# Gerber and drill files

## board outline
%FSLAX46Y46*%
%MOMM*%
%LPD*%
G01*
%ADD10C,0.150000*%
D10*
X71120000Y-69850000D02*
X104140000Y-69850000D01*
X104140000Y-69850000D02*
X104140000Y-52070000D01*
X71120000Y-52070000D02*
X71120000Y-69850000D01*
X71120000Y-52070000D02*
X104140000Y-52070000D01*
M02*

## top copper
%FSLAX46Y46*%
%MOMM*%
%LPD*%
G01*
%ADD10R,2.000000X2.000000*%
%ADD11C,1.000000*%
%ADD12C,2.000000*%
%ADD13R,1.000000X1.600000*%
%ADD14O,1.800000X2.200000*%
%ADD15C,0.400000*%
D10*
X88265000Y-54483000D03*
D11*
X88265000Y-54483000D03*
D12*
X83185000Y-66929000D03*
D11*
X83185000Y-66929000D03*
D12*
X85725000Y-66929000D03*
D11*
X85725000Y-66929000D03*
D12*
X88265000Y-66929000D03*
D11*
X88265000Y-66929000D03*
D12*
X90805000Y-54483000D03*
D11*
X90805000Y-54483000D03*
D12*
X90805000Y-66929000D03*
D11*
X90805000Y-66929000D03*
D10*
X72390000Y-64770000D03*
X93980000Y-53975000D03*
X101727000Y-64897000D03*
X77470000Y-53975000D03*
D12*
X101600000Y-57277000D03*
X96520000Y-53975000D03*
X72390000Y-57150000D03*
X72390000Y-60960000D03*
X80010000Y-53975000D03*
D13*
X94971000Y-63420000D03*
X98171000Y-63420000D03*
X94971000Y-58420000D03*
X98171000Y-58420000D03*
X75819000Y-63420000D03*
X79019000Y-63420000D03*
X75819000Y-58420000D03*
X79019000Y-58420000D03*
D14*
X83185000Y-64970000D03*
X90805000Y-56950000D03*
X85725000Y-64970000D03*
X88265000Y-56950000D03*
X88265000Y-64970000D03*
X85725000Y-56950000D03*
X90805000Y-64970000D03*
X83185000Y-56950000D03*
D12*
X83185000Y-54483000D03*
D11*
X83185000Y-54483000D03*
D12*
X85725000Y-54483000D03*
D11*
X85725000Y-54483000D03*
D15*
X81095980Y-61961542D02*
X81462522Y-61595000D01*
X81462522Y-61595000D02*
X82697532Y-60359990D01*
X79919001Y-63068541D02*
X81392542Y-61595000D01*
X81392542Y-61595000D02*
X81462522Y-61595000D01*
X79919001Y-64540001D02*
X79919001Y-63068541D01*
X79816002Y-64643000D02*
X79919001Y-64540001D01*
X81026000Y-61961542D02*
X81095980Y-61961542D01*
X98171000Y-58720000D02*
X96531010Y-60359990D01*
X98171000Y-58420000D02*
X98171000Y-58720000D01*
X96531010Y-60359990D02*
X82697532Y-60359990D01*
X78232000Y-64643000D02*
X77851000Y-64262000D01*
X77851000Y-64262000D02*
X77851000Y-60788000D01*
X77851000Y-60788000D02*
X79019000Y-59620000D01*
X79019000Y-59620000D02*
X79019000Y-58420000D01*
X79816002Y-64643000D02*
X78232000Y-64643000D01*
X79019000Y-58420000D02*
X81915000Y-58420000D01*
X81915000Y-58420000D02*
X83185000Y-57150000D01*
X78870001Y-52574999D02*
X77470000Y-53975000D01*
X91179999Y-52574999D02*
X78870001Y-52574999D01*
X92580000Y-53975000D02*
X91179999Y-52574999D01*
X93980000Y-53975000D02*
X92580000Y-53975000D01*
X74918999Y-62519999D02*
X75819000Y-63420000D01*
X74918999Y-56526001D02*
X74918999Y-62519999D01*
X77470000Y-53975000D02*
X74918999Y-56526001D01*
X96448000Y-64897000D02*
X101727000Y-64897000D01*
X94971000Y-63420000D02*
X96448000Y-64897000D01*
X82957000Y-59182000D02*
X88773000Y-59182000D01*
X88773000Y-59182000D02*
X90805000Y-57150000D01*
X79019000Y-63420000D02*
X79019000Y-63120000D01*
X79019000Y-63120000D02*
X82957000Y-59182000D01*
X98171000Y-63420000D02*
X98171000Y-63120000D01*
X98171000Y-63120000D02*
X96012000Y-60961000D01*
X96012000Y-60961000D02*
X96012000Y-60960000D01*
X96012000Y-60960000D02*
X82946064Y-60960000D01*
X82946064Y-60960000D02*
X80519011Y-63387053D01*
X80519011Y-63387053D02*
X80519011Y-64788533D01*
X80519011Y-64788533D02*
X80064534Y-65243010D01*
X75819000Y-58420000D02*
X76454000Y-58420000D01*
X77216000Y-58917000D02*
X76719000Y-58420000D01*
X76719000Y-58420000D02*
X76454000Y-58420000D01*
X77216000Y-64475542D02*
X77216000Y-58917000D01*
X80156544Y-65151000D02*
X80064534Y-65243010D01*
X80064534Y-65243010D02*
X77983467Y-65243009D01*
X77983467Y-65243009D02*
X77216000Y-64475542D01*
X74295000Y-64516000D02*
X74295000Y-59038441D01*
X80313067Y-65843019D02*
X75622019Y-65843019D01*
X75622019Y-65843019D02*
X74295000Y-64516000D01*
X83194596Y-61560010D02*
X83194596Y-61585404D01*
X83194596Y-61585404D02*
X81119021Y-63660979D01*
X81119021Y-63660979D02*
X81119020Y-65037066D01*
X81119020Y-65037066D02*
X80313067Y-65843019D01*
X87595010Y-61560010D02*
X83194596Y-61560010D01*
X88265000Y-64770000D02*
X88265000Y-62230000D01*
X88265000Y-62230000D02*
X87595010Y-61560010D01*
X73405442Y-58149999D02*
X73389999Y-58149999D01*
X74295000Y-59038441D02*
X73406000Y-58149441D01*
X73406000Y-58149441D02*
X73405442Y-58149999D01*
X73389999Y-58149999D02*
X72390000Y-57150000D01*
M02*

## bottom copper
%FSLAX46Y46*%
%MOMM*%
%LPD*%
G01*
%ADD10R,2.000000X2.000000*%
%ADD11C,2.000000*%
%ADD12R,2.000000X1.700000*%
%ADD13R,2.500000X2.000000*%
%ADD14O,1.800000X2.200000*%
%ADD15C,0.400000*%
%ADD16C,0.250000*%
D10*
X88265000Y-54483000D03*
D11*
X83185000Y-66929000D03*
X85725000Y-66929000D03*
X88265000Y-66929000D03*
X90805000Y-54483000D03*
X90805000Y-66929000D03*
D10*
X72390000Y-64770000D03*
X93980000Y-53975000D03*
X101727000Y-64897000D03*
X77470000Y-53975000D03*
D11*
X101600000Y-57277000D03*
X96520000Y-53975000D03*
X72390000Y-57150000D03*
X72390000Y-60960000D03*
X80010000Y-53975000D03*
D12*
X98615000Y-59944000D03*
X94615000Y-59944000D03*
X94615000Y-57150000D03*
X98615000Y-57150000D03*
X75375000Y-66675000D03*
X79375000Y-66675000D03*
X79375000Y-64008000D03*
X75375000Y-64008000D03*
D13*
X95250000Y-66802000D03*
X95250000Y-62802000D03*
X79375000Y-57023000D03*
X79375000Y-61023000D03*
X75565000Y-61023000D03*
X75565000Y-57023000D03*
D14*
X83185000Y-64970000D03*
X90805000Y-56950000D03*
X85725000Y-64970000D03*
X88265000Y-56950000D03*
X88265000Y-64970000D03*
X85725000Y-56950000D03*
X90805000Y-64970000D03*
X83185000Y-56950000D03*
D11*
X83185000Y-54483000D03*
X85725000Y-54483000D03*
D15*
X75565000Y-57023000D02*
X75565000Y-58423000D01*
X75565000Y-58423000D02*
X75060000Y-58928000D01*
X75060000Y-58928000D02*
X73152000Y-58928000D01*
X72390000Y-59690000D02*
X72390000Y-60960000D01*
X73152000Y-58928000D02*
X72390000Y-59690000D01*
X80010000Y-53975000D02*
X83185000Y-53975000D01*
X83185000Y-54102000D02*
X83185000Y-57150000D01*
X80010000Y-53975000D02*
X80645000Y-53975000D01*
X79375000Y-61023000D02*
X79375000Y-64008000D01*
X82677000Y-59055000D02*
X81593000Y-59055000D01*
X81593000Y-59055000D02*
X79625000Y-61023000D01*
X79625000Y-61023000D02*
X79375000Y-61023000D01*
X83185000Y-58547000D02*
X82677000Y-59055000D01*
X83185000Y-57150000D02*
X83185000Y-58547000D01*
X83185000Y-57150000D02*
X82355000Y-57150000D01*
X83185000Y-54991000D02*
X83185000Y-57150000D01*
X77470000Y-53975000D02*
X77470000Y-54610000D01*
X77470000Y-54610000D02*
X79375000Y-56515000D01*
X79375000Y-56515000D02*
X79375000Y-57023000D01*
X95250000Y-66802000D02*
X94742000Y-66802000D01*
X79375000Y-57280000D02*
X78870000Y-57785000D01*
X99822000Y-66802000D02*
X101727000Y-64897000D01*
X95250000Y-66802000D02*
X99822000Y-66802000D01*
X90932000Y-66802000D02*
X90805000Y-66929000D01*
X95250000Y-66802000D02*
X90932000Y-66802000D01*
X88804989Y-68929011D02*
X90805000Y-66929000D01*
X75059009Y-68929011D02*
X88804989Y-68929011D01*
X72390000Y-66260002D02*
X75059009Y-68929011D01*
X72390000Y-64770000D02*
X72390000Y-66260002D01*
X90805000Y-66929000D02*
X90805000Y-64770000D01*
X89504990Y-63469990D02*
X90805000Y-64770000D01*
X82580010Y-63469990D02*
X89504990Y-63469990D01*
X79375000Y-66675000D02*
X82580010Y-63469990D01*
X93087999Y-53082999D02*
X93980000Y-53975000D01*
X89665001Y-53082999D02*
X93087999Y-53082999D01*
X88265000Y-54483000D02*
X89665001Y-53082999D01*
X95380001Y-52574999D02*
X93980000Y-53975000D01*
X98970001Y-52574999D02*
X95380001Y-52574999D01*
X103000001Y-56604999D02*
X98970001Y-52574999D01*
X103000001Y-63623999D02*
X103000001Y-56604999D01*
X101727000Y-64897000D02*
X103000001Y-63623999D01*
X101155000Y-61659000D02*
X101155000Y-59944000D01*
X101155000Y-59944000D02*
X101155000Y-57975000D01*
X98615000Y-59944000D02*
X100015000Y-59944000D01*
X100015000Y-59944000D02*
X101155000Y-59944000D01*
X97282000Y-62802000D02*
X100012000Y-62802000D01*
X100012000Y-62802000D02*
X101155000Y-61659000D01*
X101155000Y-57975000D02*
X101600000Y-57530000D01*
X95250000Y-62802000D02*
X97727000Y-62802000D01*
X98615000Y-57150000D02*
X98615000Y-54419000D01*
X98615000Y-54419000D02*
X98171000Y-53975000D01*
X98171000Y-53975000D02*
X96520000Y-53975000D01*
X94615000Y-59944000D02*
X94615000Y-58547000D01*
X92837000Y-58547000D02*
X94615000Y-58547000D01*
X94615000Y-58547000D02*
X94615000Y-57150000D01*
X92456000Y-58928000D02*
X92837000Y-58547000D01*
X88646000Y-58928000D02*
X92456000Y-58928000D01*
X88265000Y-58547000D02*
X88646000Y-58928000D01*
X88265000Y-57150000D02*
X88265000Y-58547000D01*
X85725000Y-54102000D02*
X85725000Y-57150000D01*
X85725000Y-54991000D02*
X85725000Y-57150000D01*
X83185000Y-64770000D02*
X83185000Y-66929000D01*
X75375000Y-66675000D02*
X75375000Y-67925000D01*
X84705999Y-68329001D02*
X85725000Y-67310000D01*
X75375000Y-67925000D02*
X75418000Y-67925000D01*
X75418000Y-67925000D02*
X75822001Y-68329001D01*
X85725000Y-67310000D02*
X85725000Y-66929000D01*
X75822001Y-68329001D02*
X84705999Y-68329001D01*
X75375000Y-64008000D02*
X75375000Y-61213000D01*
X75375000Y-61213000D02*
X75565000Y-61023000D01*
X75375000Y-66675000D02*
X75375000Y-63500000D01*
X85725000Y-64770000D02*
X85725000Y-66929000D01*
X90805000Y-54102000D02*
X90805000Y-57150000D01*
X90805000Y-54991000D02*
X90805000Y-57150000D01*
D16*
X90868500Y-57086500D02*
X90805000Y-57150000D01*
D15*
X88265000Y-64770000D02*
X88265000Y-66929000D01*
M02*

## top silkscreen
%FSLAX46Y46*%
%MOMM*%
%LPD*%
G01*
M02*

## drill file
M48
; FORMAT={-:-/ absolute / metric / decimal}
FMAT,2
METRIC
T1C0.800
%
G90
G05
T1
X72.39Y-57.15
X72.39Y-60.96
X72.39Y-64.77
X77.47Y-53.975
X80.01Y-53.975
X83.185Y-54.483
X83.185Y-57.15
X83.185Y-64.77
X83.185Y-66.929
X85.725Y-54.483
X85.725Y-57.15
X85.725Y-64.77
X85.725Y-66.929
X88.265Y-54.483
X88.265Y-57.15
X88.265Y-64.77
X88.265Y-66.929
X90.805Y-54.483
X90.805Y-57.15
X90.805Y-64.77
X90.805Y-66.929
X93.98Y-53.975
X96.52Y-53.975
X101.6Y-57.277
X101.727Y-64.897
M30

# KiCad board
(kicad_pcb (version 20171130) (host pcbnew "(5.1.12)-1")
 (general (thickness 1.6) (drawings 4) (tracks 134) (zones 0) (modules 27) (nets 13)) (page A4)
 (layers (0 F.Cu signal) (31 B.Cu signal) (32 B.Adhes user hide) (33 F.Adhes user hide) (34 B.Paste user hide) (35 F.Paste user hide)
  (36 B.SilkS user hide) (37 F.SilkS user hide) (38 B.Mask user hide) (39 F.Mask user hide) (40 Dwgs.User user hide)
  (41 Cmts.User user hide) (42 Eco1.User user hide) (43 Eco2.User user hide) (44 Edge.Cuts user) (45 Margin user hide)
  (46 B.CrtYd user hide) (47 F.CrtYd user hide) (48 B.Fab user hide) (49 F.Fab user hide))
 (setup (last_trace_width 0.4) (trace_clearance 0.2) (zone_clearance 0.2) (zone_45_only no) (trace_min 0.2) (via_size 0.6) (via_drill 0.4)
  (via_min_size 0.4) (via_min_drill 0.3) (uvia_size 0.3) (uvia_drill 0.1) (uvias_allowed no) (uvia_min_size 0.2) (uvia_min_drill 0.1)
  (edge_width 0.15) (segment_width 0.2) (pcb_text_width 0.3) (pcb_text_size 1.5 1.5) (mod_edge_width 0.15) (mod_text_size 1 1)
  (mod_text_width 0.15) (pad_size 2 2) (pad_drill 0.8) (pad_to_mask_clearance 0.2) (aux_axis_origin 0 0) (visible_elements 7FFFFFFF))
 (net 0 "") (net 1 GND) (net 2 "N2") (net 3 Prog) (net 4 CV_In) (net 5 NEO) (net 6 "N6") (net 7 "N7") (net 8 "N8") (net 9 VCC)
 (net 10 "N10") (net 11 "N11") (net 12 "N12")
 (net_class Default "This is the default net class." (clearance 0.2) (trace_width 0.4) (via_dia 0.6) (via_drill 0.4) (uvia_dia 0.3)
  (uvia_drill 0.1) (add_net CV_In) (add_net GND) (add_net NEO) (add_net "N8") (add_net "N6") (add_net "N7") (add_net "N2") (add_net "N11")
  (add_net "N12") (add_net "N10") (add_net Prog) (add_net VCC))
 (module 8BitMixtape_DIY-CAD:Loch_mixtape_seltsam (layer F.Cu) (at 88.265 54.483)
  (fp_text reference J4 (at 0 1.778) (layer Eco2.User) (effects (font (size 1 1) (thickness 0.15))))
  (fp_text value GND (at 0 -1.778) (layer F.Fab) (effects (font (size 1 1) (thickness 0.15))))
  (pad 1 thru_hole rect (at 0 0) (size 2 2) (drill 0.8) (layers B.Cu B.Mask) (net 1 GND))
  (pad "" smd circle (at 0 0) (size 1 1) (layers F.Cu F.Paste F.Mask)))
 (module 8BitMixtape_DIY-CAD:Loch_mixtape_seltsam (layer F.Cu) (at 83.185 66.929)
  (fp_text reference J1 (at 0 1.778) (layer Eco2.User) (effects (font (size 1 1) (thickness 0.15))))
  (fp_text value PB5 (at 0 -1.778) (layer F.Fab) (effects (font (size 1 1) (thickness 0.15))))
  (pad 1 thru_hole circle (at 0 0) (size 2 2) (drill 0.8) (layers B.Cu B.Mask) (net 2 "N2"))
  (pad "" smd circle (at 0 0) (size 1 1) (layers F.Cu F.Paste F.Mask)))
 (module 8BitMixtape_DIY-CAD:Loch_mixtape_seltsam (layer F.Cu) (at 85.725 66.929)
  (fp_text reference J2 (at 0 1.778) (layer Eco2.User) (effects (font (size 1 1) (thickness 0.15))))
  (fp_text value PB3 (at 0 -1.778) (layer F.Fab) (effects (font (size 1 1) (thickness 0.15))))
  (pad 1 thru_hole circle (at 0 0) (size 2 2) (drill 0.8) (layers B.Cu B.Mask) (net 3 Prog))
  (pad "" smd circle (at 0 0) (size 1 1) (layers F.Cu F.Paste F.Mask)))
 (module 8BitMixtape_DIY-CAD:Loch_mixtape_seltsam (layer F.Cu) (at 88.265 66.929)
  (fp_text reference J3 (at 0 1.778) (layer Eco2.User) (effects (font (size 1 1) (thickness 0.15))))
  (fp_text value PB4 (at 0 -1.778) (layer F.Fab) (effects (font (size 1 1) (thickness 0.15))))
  (pad 1 thru_hole circle (at 0 0) (size 2 2) (drill 0.8) (layers B.Cu B.Mask) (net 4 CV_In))
  (pad "" smd circle (at 0 0) (size 1 1) (layers F.Cu F.Paste F.Mask)))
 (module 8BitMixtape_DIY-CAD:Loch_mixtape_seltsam (layer F.Cu) (at 90.805 54.483)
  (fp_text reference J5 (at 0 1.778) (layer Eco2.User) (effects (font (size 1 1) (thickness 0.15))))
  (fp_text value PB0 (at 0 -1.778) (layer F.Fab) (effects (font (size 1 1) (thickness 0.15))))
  (pad 1 thru_hole circle (at 0 0) (size 2 2) (drill 0.8) (layers B.Cu B.Mask) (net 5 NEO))
  (pad "" smd circle (at 0 0) (size 1 1) (layers F.Cu F.Paste F.Mask)))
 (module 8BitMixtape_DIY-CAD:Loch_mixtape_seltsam (layer F.Cu) (at 90.805 66.929)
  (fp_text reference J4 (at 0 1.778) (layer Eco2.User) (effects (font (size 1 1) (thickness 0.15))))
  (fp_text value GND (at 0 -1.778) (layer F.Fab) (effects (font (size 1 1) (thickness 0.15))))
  (pad 1 thru_hole circle (at 0 0) (size 2 2) (drill 0.8) (layers B.Cu B.Mask) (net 1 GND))
  (pad "" smd circle (at 0 0) (size 1 1) (layers F.Cu F.Paste F.Mask)))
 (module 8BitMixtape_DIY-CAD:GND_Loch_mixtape (layer F.Cu) (at 72.39 64.77)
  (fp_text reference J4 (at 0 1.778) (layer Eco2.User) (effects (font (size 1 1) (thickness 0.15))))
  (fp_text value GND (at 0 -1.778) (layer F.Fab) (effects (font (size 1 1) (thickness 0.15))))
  (pad 1 thru_hole rect (at 0 0) (size 2 2) (drill 0.8) (layers *.Cu *.Mask) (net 1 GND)))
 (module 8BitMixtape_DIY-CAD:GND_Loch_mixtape (layer F.Cu) (at 93.98 53.975)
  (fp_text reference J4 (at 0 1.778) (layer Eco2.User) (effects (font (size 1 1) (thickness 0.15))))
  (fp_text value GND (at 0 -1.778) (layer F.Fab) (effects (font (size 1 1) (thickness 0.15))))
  (pad 1 thru_hole rect (at 0 0) (size 2 2) (drill 0.8) (layers *.Cu *.Mask) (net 1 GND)))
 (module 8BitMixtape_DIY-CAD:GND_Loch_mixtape (layer F.Cu) (at 101.727 64.897)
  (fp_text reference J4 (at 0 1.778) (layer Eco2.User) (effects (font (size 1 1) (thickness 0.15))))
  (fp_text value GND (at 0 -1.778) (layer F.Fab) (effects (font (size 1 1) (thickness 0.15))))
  (pad 1 thru_hole rect (at 0 0) (size 2 2) (drill 0.8) (layers *.Cu *.Mask) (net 1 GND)))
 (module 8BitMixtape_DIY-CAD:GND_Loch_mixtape (layer F.Cu) (at 77.47 53.975)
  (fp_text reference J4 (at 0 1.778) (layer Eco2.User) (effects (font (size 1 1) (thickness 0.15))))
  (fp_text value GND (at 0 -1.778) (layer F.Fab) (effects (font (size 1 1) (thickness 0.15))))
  (pad 1 thru_hole rect (at 0 0) (size 2 2) (drill 0.8) (layers *.Cu *.Mask) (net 1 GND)))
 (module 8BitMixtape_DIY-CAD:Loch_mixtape (layer F.Cu) (at 101.6 57.277)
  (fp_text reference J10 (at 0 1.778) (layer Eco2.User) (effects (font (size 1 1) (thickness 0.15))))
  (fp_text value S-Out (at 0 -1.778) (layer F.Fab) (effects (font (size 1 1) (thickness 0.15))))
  (pad 1 thru_hole circle (at 0 0) (size 2 2) (drill 0.8) (layers *.Cu *.Mask) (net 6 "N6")))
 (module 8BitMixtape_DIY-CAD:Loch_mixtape (layer F.Cu) (at 96.52 53.975)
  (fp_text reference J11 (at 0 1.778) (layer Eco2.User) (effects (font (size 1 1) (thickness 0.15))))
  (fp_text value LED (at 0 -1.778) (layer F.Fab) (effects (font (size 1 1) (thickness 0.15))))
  (pad 1 thru_hole circle (at 0 0) (size 2 2) (drill 0.8) (layers *.Cu *.Mask) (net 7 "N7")))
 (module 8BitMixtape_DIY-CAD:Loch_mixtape (layer F.Cu) (at 72.39 57.15)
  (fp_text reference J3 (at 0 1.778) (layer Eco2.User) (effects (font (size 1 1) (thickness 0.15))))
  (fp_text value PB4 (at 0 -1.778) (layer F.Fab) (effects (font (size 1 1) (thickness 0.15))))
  (pad 1 thru_hole circle (at 0 0) (size 2 2) (drill 0.8) (layers *.Cu *.Mask) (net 4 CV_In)))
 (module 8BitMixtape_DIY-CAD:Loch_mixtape (layer F.Cu) (at 72.39 60.96)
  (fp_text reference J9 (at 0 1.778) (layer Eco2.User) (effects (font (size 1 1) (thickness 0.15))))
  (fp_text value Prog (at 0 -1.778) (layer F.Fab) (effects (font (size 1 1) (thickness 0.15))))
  (pad 1 thru_hole circle (at 0 0) (size 2 2) (drill 0.8) (layers *.Cu *.Mask) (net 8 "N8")))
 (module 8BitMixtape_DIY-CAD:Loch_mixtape (layer F.Cu) (at 80.01 53.975)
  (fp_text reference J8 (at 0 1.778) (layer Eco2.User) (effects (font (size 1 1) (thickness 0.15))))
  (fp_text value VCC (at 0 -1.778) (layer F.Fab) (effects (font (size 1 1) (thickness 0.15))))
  (pad 1 thru_hole circle (at 0 0) (size 2 2) (drill 0.8) (layers *.Cu *.Mask) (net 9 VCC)))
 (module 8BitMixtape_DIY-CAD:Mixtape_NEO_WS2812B (layer F.Cu) (at 96.571 60.92 270)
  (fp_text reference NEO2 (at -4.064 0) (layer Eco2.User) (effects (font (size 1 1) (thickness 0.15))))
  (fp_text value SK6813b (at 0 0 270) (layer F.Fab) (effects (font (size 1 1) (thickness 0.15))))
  (pad 3 smd rect (at 2.5 1.6 270) (size 1.6 1) (layers F.Cu F.Paste F.Mask) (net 1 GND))
  (pad 4 smd rect (at 2.5 -1.6 270) (size 1.6 1) (layers F.Cu F.Paste F.Mask) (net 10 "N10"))
  (pad 2 smd rect (at -2.5 1.6 270) (size 1.6 1) (layers F.Cu F.Paste F.Mask))
  (pad 1 smd rect (at -2.5 -1.6 270) (size 1.6 1) (layers F.Cu F.Paste F.Mask) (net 9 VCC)))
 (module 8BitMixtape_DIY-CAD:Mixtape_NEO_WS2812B (layer F.Cu) (at 77.419 60.92 270)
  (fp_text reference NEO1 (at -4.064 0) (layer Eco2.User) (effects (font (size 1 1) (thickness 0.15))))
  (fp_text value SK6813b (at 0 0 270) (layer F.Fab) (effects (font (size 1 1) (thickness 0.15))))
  (pad 3 smd rect (at 2.5 1.6 270) (size 1.6 1) (layers F.Cu F.Paste F.Mask) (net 1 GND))
  (pad 4 smd rect (at 2.5 -1.6 270) (size 1.6 1) (layers F.Cu F.Paste F.Mask) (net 5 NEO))
  (pad 2 smd rect (at -2.5 1.6 270) (size 1.6 1) (layers F.Cu F.Paste F.Mask) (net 10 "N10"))
  (pad 1 smd rect (at -2.5 -1.6 270) (size 1.6 1) (layers F.Cu F.Paste F.Mask) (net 9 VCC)))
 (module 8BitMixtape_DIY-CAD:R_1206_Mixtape (layer B.Cu) (at 96.615 59.944 180)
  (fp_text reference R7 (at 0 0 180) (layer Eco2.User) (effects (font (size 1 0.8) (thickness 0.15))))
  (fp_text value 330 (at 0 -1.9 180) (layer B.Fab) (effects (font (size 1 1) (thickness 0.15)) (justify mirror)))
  (pad 1 smd rect (at -2 0 180) (size 2 1.7) (layers B.Cu B.Paste B.Mask) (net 6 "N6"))
  (pad 2 smd rect (at 2 0 180) (size 2 1.7) (layers B.Cu B.Paste B.Mask) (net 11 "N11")))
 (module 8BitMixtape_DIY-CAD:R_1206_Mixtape (layer B.Cu) (at 96.615 57.15)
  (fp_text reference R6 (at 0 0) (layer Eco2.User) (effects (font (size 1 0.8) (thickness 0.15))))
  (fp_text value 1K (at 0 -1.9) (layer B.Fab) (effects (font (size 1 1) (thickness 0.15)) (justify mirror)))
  (pad 1 smd rect (at -2 0) (size 2 1.7) (layers B.Cu B.Paste B.Mask) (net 11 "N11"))
  (pad 2 smd rect (at 2 0) (size 2 1.7) (layers B.Cu B.Paste B.Mask) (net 7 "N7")))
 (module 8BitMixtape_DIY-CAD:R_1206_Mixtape (layer B.Cu) (at 77.375 66.675)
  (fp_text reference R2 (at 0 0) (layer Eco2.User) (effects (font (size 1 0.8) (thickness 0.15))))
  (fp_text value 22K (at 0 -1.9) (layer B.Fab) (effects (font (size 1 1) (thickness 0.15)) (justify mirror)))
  (pad 1 smd rect (at -2 0) (size 2 1.7) (layers B.Cu B.Paste B.Mask) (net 3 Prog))
  (pad 2 smd rect (at 2 0) (size 2 1.7) (layers B.Cu B.Paste B.Mask) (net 1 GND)))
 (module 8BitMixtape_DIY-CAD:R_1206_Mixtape (layer B.Cu) (at 77.375 64.008 180)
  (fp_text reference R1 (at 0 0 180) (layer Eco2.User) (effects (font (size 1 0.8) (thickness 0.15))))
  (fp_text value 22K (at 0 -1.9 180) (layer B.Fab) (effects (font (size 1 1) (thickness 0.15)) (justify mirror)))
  (pad 1 smd rect (at -2 0 180) (size 2 1.7) (layers B.Cu B.Paste B.Mask) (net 9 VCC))
  (pad 2 smd rect (at 2 0 180) (size 2 1.7) (layers B.Cu B.Paste B.Mask) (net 3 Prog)))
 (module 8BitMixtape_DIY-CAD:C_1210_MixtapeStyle (layer B.Cu) (at 95.25 64.802 90)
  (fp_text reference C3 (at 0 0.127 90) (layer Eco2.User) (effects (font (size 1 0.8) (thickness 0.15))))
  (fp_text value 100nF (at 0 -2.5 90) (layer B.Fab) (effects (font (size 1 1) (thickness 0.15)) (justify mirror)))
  (pad 1 smd rect (at -2 0 90) (size 2 2.5) (layers B.Cu B.Paste B.Mask) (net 1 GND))
  (pad 2 smd rect (at 2 0 90) (size 2 2.5) (layers B.Cu B.Paste B.Mask) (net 6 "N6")))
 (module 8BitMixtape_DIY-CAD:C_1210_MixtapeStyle (layer B.Cu) (at 79.375 59.023 270)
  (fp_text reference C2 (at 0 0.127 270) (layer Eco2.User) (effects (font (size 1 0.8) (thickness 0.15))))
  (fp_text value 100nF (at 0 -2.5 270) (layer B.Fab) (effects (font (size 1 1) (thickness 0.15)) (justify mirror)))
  (pad 1 smd rect (at -2 0 270) (size 2 2.5) (layers B.Cu B.Paste B.Mask) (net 1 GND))
  (pad 2 smd rect (at 2 0 270) (size 2 2.5) (layers B.Cu B.Paste B.Mask) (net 9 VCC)))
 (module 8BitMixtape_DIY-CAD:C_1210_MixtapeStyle (layer B.Cu) (at 75.565 59.023 90)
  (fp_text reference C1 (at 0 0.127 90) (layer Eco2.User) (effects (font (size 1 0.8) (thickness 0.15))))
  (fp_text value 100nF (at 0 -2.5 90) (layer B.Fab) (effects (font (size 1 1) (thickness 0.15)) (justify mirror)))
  (pad 1 smd rect (at -2 0 90) (size 2 2.5) (layers B.Cu B.Paste B.Mask) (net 3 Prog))
  (pad 2 smd rect (at 2 0 90) (size 2 2.5) (layers B.Cu B.Paste B.Mask) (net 8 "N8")))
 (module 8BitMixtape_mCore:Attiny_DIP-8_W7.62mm (layer F.Cu) (at 83.185 64.77 90)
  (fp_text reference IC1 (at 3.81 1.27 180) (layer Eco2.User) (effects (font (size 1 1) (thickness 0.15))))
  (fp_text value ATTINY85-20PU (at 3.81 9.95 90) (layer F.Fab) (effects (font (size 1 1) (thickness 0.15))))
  (pad 1 thru_hole oval (at 0 0 90) (size 2.2 1.8) (drill 0.8 (offset -0.2 0)) (layers *.Cu *.Mask) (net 2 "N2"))
  (pad 5 thru_hole oval (at 7.62 7.62 90) (size 2.2 1.8) (drill 0.8 (offset 0.2 0)) (layers *.Cu *.Mask) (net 5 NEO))
  (pad 2 thru_hole oval (at 0 2.54 90) (size 2.2 1.8) (drill 0.8 (offset -0.2 0)) (layers *.Cu *.Mask) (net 3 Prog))
  (pad 6 thru_hole oval (at 7.62 5.08 90) (size 2.2 1.8) (drill 0.8 (offset 0.2 0)) (layers *.Cu *.Mask) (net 11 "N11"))
  (pad 3 thru_hole oval (at 0 5.08 90) (size 2.2 1.8) (drill 0.8 (offset -0.2 0)) (layers *.Cu *.Mask) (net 4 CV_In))
  (pad 7 thru_hole oval (at 7.62 2.54 90) (size 2.2 1.8) (drill 0.8 (offset 0.2 0)) (layers *.Cu *.Mask) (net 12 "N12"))
  (pad 4 thru_hole oval (at 0 7.62 90) (size 2.2 1.8) (drill 0.8 (offset -0.2 0)) (layers *.Cu *.Mask) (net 1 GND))
  (pad 8 thru_hole oval (at 7.62 0 90) (size 2.2 1.8) (drill 0.8 (offset 0.2 0)) (layers *.Cu *.Mask) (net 9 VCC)))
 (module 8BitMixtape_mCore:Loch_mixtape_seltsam (layer F.Cu) (at 83.185 54.483)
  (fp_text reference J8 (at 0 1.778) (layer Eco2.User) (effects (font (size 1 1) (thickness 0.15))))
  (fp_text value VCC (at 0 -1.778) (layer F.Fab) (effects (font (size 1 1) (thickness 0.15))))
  (pad 1 thru_hole circle (at 0 0) (size 2 2) (drill 0.8) (layers B.Cu B.Mask) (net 9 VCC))
  (pad "" smd circle (at 0 0) (size 1 1) (layers F.Cu F.Paste F.Mask)))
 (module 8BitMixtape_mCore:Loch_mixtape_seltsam (layer F.Cu) (at 85.725 54.483)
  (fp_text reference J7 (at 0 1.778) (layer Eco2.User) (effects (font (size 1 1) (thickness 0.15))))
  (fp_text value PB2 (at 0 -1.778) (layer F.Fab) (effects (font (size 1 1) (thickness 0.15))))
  (pad 1 thru_hole circle (at 0 0) (size 2 2) (drill 0.8) (layers B.Cu B.Mask) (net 12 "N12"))
  (pad "" smd circle (at 0 0) (size 1 1) (layers F.Cu F.Paste F.Mask)))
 (gr_line (start 71.12 69.85) (end 104.14 69.85) (layer Edge.Cuts) (width 0.15))
 (gr_line (start 104.14 69.85) (end 104.14 52.07) (layer Edge.Cuts) (width 0.15))
 (gr_line (start 71.12 52.07) (end 71.12 69.85) (layer Edge.Cuts) (width 0.15))
 (gr_line (start 71.12 52.07) (end 104.14 52.07) (layer Edge.Cuts) (width 0.15))
 (segment (start 75.565 57.023) (end 75.565 58.423) (width 0.4) (layer B.Cu) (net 8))
 (segment (start 75.565 58.423) (end 75.06 58.928) (width 0.4) (layer B.Cu) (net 8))
 (segment (start 75.06 58.928) (end 73.152 58.928) (width 0.4) (layer B.Cu) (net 8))
 (segment (start 72.39 59.69) (end 72.39 60.96) (width 0.4) (layer B.Cu) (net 8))
 (segment (start 73.152 58.928) (end 72.39 59.69) (width 0.4) (layer B.Cu) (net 8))
 (segment (start 81.09598 61.961542) (end 81.462522 61.595) (width 0.4) (layer F.Cu) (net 9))
 (segment (start 81.462522 61.595) (end 82.697532 60.35999) (width 0.4) (layer F.Cu) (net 9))
 (segment (start 79.919001 63.068541) (end 81.392542 61.595) (width 0.4) (layer F.Cu) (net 9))
 (segment (start 81.392542 61.595) (end 81.462522 61.595) (width 0.4) (layer F.Cu) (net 9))
 (segment (start 79.919001 64.540001) (end 79.919001 63.068541) (width 0.4) (layer F.Cu) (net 9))
 (segment (start 79.816002 64.643) (end 79.919001 64.540001) (width 0.4) (layer F.Cu) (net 9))
 (segment (start 81.026 61.961542) (end 81.09598 61.961542) (width 0.4) (layer F.Cu) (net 9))
 (segment (start 98.171 58.72) (end 96.53101 60.35999) (width 0.4) (layer F.Cu) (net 9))
 (segment (start 98.171 58.42) (end 98.171 58.72) (width 0.4) (layer F.Cu) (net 9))
 (segment (start 96.53101 60.35999) (end 82.697532 60.35999) (width 0.4) (layer F.Cu) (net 9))
 (segment (start 78.232 64.643) (end 77.851 64.262) (width 0.4) (layer F.Cu) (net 9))
 (segment (start 77.851 64.262) (end 77.851 60.788) (width 0.4) (layer F.Cu) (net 9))
 (segment (start 77.851 60.788) (end 79.019 59.62) (width 0.4) (layer F.Cu) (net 9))
 (segment (start 79.019 59.62) (end 79.019 58.42) (width 0.4) (layer F.Cu) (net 9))
 (segment (start 79.816002 64.643) (end 78.232 64.643) (width 0.4) (layer F.Cu) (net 9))
 (segment (start 79.019 58.42) (end 81.915 58.42) (width 0.4) (layer F.Cu) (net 9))
 (segment (start 81.915 58.42) (end 83.185 57.15) (width 0.4) (layer F.Cu) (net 9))
 (segment (start 80.01 53.975) (end 83.185 53.975) (width 0.4) (layer B.Cu) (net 9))
 (segment (start 83.185 54.102) (end 83.185 57.15) (width 0.4) (layer B.Cu) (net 9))
 (segment (start 80.01 53.975) (end 80.645 53.975) (width 0.4) (layer B.Cu) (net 9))
 (segment (start 79.375 61.023) (end 79.375 64.008) (width 0.4) (layer B.Cu) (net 9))
 (segment (start 82.677 59.055) (end 81.593 59.055) (width 0.4) (layer B.Cu) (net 9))
 (segment (start 81.593 59.055) (end 79.625 61.023) (width 0.4) (layer B.Cu) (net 9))
 (segment (start 79.625 61.023) (end 79.375 61.023) (width 0.4) (layer B.Cu) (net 9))
 (segment (start 83.185 58.547) (end 82.677 59.055) (width 0.4) (layer B.Cu) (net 9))
 (segment (start 83.185 57.15) (end 83.185 58.547) (width 0.4) (layer B.Cu) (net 9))
 (segment (start 83.185 57.15) (end 82.355 57.15) (width 0.4) (layer B.Cu) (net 9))
 (segment (start 83.185 54.991) (end 83.185 57.15) (width 0.4) (layer B.Cu) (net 9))
 (segment (start 77.47 53.975) (end 77.47 54.61) (width 0.4) (layer B.Cu) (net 1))
 (segment (start 77.47 54.61) (end 79.375 56.515) (width 0.4) (layer B.Cu) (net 1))
 (segment (start 79.375 56.515) (end 79.375 57.023) (width 0.4) (layer B.Cu) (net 1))
 (segment (start 95.25 66.802) (end 94.742 66.802) (width 0.4) (layer B.Cu) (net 1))
 (segment (start 79.375 57.28) (end 78.87 57.785) (width 0.4) (layer B.Cu) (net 1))
 (segment (start 78.870001 52.574999) (end 77.47 53.975) (width 0.4) (layer F.Cu) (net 1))
 (segment (start 91.179999 52.574999) (end 78.870001 52.574999) (width 0.4) (layer F.Cu) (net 1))
 (segment (start 92.58 53.975) (end 91.179999 52.574999) (width 0.4) (layer F.Cu) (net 1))
 (segment (start 93.98 53.975) (end 92.58 53.975) (width 0.4) (layer F.Cu) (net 1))
 (segment (start 74.918999 62.519999) (end 75.819 63.42) (width 0.4) (layer F.Cu) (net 1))
 (segment (start 74.918999 56.526001) (end 74.918999 62.519999) (width 0.4) (layer F.Cu) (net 1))
 (segment (start 77.47 53.975) (end 74.918999 56.526001) (width 0.4) (layer F.Cu) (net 1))
 (segment (start 96.448 64.897) (end 101.727 64.897) (width 0.4) (layer F.Cu) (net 1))
 (segment (start 94.971 63.42) (end 96.448 64.897) (width 0.4) (layer F.Cu) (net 1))
 (segment (start 99.822 66.802) (end 101.727 64.897) (width 0.4) (layer B.Cu) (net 1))
 (segment (start 95.25 66.802) (end 99.822 66.802) (width 0.4) (layer B.Cu) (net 1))
 (segment (start 90.932 66.802) (end 90.805 66.929) (width 0.4) (layer B.Cu) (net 1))
 (segment (start 95.25 66.802) (end 90.932 66.802) (width 0.4) (layer B.Cu) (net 1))
 (segment (start 88.804989 68.929011) (end 90.805 66.929) (width 0.4) (layer B.Cu) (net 1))
 (segment (start 75.059009 68.929011) (end 88.804989 68.929011) (width 0.4) (layer B.Cu) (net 1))
 (segment (start 72.39 66.260002) (end 75.059009 68.929011) (width 0.4) (layer B.Cu) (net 1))
 (segment (start 72.39 64.77) (end 72.39 66.260002) (width 0.4) (layer B.Cu) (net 1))
 (segment (start 90.805 66.929) (end 90.805 64.77) (width 0.4) (layer B.Cu) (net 1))
 (segment (start 89.50499 63.46999) (end 90.805 64.77) (width 0.4) (layer B.Cu) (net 1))
 (segment (start 82.58001 63.46999) (end 89.50499 63.46999) (width 0.4) (layer B.Cu) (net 1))
 (segment (start 79.375 66.675) (end 82.58001 63.46999) (width 0.4) (layer B.Cu) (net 1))
 (segment (start 93.087999 53.082999) (end 93.98 53.975) (width 0.4) (layer B.Cu) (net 1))
 (segment (start 89.665001 53.082999) (end 93.087999 53.082999) (width 0.4) (layer B.Cu) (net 1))
 (segment (start 88.265 54.483) (end 89.665001 53.082999) (width 0.4) (layer B.Cu) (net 1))
 (segment (start 95.380001 52.574999) (end 93.98 53.975) (width 0.4) (layer B.Cu) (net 1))
 (segment (start 98.970001 52.574999) (end 95.380001 52.574999) (width 0.4) (layer B.Cu) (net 1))
 (segment (start 103.000001 56.604999) (end 98.970001 52.574999) (width 0.4) (layer B.Cu) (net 1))
 (segment (start 103.000001 63.623999) (end 103.000001 56.604999) (width 0.4) (layer B.Cu) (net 1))
 (segment (start 101.727 64.897) (end 103.000001 63.623999) (width 0.4) (layer B.Cu) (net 1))
 (segment (start 101.155 61.659) (end 101.155 59.944) (width 0.4) (layer B.Cu) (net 6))
 (segment (start 101.155 59.944) (end 101.155 57.975) (width 0.4) (layer B.Cu) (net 6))
 (segment (start 98.615 59.944) (end 100.015 59.944) (width 0.4) (layer B.Cu) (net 6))
 (segment (start 100.015 59.944) (end 101.155 59.944) (width 0.4) (layer B.Cu) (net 6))
 (segment (start 97.282 62.802) (end 100.012 62.802) (width 0.4) (layer B.Cu) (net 6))
 (segment (start 100.012 62.802) (end 101.155 61.659) (width 0.4) (layer B.Cu) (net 6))
 (segment (start 101.155 57.975) (end 101.6 57.53) (width 0.4) (layer B.Cu) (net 6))
 (segment (start 95.25 62.802) (end 97.727 62.802) (width 0.4) (layer B.Cu) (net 6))
 (segment (start 98.615 57.15) (end 98.615 54.419) (width 0.4) (layer B.Cu) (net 7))
 (segment (start 98.615 54.419) (end 98.171 53.975) (width 0.4) (layer B.Cu) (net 7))
 (segment (start 98.171 53.975) (end 96.52 53.975) (width 0.4) (layer B.Cu) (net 7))
 (segment (start 94.615 59.944) (end 94.615 58.547) (width 0.4) (layer B.Cu) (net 11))
 (segment (start 92.837 58.547) (end 94.615 58.547) (width 0.4) (layer B.Cu) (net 11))
 (segment (start 94.615 58.547) (end 94.615 57.15) (width 0.4) (layer B.Cu) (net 11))
 (segment (start 92.456 58.928) (end 92.837 58.547) (width 0.4) (layer B.Cu) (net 11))
 (segment (start 88.646 58.928) (end 92.456 58.928) (width 0.4) (layer B.Cu) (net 11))
 (segment (start 88.265 58.547) (end 88.646 58.928) (width 0.4) (layer B.Cu) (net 11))
 (segment (start 88.265 57.15) (end 88.265 58.547) (width 0.4) (layer B.Cu) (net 11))
 (segment (start 85.725 54.102) (end 85.725 57.15) (width 0.4) (layer B.Cu) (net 12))
 (segment (start 85.725 54.991) (end 85.725 57.15) (width 0.4) (layer B.Cu) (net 12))
 (segment (start 83.185 64.77) (end 83.185 66.929) (width 0.4) (layer B.Cu) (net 2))
 (segment (start 75.375 66.675) (end 75.375 67.925) (width 0.4) (layer B.Cu) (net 3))
 (segment (start 84.705999 68.329001) (end 85.725 67.31) (width 0.4) (layer B.Cu) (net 3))
 (segment (start 75.375 67.925) (end 75.418 67.925) (width 0.4) (layer B.Cu) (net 3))
 (segment (start 75.418 67.925) (end 75.822001 68.329001) (width 0.4) (layer B.Cu) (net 3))
 (segment (start 85.725 67.31) (end 85.725 66.929) (width 0.4) (layer B.Cu) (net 3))
 (segment (start 75.822001 68.329001) (end 84.705999 68.329001) (width 0.4) (layer B.Cu) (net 3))
 (segment (start 75.375 64.008) (end 75.375 61.213) (width 0.4) (layer B.Cu) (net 3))
 (segment (start 75.375 61.213) (end 75.565 61.023) (width 0.4) (layer B.Cu) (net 3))
 (segment (start 75.375 66.675) (end 75.375 63.5) (width 0.4) (layer B.Cu) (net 3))
 (segment (start 85.725 64.77) (end 85.725 66.929) (width 0.4) (layer B.Cu) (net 3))
 (segment (start 82.957 59.182) (end 88.773 59.182) (width 0.4) (layer F.Cu) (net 5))
 (segment (start 88.773 59.182) (end 90.805 57.15) (width 0.4) (layer F.Cu) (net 5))
 (segment (start 79.019 63.42) (end 79.019 63.12) (width 0.4) (layer F.Cu) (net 5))
 (segment (start 79.019 63.12) (end 82.957 59.182) (width 0.4) (layer F.Cu) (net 5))
 (segment (start 90.805 54.102) (end 90.805 57.15) (width 0.4) (layer B.Cu) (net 5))
 (segment (start 90.805 54.991) (end 90.805 57.15) (width 0.4) (layer B.Cu) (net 5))
 (segment (start 90.8685 57.0865) (end 90.805 57.15) (width 0.25) (layer B.Cu) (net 5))
 (segment (start 98.171 63.42) (end 98.171 63.12) (width 0.4) (layer F.Cu) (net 10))
 (segment (start 98.171 63.12) (end 96.012 60.961) (width 0.4) (layer F.Cu) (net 10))
 (segment (start 96.012 60.961) (end 96.012 60.96) (width 0.4) (layer F.Cu) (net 10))
 (segment (start 96.012 60.96) (end 82.946064 60.96) (width 0.4) (layer F.Cu) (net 10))
 (segment (start 82.946064 60.96) (end 80.519011 63.387053) (width 0.4) (layer F.Cu) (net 10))
 (segment (start 80.519011 63.387053) (end 80.519011 64.788533) (width 0.4) (layer F.Cu) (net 10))
 (segment (start 80.519011 64.788533) (end 80.064534 65.24301) (width 0.4) (layer F.Cu) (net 10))
 (segment (start 75.819 58.42) (end 76.454 58.42) (width 0.4) (layer F.Cu) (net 10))
 (segment (start 77.216 58.917) (end 76.719 58.42) (width 0.4) (layer F.Cu) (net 10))
 (segment (start 76.719 58.42) (end 76.454 58.42) (width 0.4) (layer F.Cu) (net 10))
 (segment (start 77.216 64.475542) (end 77.216 58.917) (width 0.4) (layer F.Cu) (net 10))
 (segment (start 80.156544 65.151) (end 80.064534 65.24301) (width 0.4) (layer F.Cu) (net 10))
 (segment (start 80.064534 65.24301) (end 77.983467 65.243009) (width 0.4) (layer F.Cu) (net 10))
 (segment (start 77.983467 65.243009) (end 77.216 64.475542) (width 0.4) (layer F.Cu) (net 10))
 (segment (start 74.295 64.516) (end 74.295 59.038441) (width 0.4) (layer F.Cu) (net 4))
 (segment (start 80.313067 65.843019) (end 75.622019 65.843019) (width 0.4) (layer F.Cu) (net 4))
 (segment (start 75.622019 65.843019) (end 74.295 64.516) (width 0.4) (layer F.Cu) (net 4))
 (segment (start 83.194596 61.56001) (end 83.194596 61.585404) (width 0.4) (layer F.Cu) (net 4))
 (segment (start 83.194596 61.585404) (end 81.119021 63.660979) (width 0.4) (layer F.Cu) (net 4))
 (segment (start 81.119021 63.660979) (end 81.11902 65.037066) (width 0.4) (layer F.Cu) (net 4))
 (segment (start 81.11902 65.037066) (end 80.313067 65.843019) (width 0.4) (layer F.Cu) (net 4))
 (segment (start 87.59501 61.56001) (end 83.194596 61.56001) (width 0.4) (layer F.Cu) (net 4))
 (segment (start 88.265 64.77) (end 88.265 62.23) (width 0.4) (layer F.Cu) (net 4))
 (segment (start 88.265 62.23) (end 87.59501 61.56001) (width 0.4) (layer F.Cu) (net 4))
 (segment (start 73.405442 58.149999) (end 73.389999 58.149999) (width 0.4) (layer F.Cu) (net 4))
 (segment (start 74.295 59.038441) (end 73.406 58.149441) (width 0.4) (layer F.Cu) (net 4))
 (segment (start 73.406 58.149441) (end 73.405442 58.149999) (width 0.4) (layer F.Cu) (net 4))
 (segment (start 73.389999 58.149999) (end 72.39 57.15) (width 0.4) (layer F.Cu) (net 4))
 (segment (start 88.265 64.77) (end 88.265 66.929) (width 0.4) (layer B.Cu) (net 4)))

